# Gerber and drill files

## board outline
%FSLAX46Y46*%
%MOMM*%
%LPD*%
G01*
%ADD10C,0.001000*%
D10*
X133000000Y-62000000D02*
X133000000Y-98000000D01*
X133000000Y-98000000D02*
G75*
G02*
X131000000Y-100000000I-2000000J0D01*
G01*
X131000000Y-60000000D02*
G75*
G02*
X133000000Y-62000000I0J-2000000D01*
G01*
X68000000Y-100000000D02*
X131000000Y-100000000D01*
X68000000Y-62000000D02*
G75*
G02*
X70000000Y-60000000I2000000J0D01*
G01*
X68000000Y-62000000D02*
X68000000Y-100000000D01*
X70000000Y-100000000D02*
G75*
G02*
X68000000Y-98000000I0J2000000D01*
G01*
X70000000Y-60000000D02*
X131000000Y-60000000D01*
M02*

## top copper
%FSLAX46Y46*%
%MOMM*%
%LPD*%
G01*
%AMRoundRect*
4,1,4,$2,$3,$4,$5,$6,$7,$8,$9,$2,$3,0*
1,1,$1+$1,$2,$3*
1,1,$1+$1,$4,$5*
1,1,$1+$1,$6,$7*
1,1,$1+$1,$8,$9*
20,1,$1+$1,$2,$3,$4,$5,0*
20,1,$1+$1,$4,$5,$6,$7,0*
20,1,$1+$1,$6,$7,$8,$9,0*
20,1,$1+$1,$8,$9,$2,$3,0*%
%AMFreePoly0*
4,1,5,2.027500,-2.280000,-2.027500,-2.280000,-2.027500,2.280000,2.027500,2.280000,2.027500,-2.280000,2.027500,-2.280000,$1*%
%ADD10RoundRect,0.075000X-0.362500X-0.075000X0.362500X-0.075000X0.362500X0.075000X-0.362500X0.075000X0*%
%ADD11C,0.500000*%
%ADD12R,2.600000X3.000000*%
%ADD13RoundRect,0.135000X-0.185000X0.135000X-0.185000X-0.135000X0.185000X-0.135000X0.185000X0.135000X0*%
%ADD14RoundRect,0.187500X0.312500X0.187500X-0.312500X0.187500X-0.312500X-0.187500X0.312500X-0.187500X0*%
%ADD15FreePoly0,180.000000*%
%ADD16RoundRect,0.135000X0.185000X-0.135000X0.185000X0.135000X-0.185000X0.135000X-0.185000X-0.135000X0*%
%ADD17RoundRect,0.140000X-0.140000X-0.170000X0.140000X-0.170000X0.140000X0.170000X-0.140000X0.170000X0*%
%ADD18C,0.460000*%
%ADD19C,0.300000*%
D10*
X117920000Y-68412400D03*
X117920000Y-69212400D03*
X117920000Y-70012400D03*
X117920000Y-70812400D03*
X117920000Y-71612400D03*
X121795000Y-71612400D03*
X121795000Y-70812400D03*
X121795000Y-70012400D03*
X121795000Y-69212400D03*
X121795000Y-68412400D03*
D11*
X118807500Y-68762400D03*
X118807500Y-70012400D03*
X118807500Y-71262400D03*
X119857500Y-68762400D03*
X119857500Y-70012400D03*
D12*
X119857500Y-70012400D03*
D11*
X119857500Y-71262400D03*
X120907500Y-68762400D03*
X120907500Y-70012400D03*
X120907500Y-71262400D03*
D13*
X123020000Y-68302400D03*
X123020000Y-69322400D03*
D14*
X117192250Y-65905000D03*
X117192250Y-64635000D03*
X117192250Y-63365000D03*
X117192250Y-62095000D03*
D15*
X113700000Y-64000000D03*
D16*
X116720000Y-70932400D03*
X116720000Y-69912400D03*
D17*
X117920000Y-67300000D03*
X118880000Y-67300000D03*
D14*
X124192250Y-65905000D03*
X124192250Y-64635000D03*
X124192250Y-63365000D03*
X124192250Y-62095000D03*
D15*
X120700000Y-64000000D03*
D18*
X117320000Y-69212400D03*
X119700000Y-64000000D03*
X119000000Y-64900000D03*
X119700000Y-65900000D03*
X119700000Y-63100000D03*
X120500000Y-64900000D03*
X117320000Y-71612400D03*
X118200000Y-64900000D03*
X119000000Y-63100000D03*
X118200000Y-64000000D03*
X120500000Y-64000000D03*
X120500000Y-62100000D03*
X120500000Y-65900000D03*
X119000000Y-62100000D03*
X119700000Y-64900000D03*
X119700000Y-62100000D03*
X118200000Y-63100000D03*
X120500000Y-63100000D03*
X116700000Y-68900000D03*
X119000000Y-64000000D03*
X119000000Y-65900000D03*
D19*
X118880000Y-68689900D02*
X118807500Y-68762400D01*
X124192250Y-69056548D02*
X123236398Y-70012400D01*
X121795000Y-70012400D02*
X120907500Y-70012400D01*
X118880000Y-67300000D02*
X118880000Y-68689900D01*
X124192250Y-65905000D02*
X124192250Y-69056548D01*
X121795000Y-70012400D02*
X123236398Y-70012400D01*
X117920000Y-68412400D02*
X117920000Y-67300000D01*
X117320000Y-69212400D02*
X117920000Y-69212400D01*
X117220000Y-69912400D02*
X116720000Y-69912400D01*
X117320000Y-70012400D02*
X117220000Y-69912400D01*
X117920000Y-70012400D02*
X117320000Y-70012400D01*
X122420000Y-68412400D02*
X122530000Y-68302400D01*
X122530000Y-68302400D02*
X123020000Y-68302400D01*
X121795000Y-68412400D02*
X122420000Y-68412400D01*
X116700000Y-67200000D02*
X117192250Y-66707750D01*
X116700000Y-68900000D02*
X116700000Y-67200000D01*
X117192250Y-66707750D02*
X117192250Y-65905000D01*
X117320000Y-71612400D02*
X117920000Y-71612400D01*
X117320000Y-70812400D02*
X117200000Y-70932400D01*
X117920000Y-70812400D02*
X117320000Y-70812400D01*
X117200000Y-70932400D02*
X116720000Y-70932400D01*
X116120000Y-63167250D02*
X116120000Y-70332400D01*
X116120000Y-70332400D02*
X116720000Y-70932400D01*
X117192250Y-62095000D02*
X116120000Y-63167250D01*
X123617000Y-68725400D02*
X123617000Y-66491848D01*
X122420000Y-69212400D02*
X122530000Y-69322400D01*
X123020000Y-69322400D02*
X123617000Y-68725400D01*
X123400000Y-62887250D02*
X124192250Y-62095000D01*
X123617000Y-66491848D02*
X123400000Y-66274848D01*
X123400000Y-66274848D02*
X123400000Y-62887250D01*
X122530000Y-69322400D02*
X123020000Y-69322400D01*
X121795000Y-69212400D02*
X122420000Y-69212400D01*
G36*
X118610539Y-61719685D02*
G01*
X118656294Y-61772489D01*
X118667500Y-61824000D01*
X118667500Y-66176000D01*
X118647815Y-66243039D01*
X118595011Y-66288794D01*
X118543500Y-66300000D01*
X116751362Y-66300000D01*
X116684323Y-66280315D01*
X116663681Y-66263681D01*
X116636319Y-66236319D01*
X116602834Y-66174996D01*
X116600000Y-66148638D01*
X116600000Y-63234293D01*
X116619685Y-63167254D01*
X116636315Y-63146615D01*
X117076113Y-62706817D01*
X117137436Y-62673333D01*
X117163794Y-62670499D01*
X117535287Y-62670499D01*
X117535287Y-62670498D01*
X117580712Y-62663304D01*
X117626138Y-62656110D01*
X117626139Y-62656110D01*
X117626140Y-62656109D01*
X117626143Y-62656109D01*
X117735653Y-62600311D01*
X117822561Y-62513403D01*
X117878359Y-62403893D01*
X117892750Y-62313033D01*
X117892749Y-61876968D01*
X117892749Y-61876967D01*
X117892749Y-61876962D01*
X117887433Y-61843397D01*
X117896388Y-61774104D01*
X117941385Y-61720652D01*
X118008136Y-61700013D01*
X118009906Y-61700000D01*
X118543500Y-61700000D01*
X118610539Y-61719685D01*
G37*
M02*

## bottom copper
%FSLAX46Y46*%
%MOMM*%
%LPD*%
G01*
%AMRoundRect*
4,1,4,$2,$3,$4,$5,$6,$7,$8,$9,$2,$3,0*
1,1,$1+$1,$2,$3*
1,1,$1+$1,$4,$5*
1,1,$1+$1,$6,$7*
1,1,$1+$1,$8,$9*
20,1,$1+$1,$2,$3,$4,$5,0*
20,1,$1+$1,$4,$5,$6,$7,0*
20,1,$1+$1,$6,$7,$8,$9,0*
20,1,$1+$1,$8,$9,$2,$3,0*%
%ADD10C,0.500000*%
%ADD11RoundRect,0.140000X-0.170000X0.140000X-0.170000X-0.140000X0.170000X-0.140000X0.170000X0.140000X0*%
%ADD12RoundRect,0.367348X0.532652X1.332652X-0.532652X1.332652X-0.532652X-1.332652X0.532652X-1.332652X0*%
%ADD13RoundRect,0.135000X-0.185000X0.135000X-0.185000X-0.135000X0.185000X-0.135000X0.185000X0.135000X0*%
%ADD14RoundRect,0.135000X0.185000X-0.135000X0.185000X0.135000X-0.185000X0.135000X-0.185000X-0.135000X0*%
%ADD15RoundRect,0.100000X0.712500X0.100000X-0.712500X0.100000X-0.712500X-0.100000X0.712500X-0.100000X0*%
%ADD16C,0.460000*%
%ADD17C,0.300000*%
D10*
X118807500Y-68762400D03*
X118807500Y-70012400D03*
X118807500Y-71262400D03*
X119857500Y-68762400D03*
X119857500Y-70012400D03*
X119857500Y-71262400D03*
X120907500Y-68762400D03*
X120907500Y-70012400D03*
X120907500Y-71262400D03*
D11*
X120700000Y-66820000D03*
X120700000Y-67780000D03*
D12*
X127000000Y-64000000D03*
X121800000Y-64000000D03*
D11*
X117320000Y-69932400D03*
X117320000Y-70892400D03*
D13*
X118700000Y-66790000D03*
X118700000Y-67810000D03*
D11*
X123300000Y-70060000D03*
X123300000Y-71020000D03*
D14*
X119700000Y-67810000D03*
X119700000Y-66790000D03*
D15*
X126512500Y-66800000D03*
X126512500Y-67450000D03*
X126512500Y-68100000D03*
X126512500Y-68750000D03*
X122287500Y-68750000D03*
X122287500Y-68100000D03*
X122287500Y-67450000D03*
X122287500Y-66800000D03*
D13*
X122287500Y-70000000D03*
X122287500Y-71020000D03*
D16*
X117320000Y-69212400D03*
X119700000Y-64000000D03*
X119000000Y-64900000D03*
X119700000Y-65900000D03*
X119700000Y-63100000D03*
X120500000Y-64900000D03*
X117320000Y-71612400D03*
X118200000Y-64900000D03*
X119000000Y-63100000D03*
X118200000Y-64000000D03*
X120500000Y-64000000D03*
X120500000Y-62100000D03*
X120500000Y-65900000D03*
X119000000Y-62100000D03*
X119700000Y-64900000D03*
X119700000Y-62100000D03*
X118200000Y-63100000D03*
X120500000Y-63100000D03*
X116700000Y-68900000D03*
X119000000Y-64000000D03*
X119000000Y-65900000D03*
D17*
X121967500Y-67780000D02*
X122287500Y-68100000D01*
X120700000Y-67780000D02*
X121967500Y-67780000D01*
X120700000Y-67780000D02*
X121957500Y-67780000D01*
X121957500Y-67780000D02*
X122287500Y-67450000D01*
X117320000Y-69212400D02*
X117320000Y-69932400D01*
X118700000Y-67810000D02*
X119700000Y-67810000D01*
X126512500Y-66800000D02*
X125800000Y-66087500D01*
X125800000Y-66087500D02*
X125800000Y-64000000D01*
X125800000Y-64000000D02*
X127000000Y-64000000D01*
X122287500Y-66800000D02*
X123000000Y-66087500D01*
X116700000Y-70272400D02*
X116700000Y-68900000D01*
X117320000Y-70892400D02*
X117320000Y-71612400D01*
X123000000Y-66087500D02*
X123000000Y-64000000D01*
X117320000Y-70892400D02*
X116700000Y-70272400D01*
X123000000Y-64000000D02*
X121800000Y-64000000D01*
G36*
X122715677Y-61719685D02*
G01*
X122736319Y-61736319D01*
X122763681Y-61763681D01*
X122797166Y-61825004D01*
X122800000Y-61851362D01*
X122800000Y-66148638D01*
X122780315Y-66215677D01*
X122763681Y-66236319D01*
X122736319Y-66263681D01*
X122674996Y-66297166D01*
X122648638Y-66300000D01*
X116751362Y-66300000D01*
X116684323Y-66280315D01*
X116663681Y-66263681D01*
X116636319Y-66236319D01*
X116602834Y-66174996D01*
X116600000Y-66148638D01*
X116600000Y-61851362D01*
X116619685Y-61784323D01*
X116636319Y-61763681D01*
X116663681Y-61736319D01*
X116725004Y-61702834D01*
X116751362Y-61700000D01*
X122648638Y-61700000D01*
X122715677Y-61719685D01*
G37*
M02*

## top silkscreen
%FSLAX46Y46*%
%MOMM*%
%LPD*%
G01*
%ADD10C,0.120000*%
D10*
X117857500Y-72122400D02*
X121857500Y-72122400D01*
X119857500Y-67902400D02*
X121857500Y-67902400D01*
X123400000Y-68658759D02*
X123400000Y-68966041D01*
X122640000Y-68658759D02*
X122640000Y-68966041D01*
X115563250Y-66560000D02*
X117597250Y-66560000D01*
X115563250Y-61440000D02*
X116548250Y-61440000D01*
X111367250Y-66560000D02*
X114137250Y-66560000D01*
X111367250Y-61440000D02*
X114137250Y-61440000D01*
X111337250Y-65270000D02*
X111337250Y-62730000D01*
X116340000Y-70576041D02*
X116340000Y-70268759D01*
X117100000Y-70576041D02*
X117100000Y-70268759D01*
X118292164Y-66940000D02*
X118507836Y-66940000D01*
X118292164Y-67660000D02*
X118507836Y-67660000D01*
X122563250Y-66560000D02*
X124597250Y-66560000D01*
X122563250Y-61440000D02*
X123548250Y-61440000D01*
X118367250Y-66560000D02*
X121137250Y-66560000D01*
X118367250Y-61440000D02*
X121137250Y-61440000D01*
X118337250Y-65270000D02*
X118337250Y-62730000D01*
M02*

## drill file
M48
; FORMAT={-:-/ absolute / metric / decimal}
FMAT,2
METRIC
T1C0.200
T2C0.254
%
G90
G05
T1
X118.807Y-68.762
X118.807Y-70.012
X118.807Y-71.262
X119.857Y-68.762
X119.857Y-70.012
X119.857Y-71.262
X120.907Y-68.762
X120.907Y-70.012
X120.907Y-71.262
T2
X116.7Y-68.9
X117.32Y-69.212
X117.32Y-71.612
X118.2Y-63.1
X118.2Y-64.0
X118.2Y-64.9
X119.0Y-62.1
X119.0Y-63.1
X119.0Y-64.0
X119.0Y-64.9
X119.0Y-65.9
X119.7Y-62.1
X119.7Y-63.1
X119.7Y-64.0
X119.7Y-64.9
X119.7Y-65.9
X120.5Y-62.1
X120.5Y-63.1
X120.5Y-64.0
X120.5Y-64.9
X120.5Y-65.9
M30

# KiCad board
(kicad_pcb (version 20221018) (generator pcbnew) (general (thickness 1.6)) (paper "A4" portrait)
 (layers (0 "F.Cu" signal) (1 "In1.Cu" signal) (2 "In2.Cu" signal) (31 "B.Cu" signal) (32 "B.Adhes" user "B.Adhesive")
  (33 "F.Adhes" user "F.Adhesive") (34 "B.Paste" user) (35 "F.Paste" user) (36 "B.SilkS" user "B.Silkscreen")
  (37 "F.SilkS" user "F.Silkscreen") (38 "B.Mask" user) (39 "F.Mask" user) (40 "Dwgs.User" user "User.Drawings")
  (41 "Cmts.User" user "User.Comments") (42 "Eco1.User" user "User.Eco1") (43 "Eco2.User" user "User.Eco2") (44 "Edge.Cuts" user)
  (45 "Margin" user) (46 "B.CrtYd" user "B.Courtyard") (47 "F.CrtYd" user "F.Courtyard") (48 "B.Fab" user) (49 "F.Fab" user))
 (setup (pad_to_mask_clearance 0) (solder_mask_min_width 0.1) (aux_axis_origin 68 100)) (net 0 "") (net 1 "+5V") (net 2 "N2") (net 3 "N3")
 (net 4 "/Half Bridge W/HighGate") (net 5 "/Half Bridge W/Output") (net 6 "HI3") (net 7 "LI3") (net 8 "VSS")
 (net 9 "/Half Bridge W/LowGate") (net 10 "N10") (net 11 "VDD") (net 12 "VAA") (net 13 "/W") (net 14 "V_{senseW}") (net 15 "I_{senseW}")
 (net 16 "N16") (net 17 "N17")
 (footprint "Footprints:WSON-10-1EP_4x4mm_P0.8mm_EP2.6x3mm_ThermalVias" (layer "F.Cu") (at 119.8575 70.0124)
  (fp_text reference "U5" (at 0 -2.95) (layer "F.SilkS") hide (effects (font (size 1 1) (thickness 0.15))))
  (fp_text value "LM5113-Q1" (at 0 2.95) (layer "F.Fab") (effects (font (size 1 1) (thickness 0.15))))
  (fp_line (start -2 2.11) (end 2 2.11) (stroke (width 0.12) (type solid)) (layer "F.SilkS"))
  (fp_line (start 0 -2.11) (end 2 -2.11) (stroke (width 0.12) (type solid)) (layer "F.SilkS"))
  (pad "" smd roundrect (at -0.65 -0.75) (size 1.05 1.21) (layers "F.Paste") (roundrect_rratio 0.238095))
  (pad "" smd roundrect (at -0.65 0.75) (size 1.05 1.21) (layers "F.Paste") (roundrect_rratio 0.238095))
  (pad "" smd roundrect (at 0.65 -0.75) (size 1.05 1.21) (layers "F.Paste") (roundrect_rratio 0.238095))
  (pad "" smd roundrect (at 0.65 0.75) (size 1.05 1.21) (layers "F.Paste") (roundrect_rratio 0.238095))
  (pad "1" smd roundrect (at -1.9375 -1.6) (size 0.875 0.3) (layers "F.Cu" "F.Paste" "F.Mask") (roundrect_rratio 0.25) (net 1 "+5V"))
  (pad "2" smd roundrect (at -1.9375 -0.8) (size 0.875 0.3) (layers "F.Cu" "F.Paste" "F.Mask") (roundrect_rratio 0.25) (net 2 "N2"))
  (pad "3" smd roundrect (at -1.9375 0) (size 0.875 0.3) (layers "F.Cu" "F.Paste" "F.Mask") (roundrect_rratio 0.25) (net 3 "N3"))
  (pad "4" smd roundrect (at -1.9375 0.8) (size 0.875 0.3) (layers "F.Cu" "F.Paste" "F.Mask") (roundrect_rratio 0.25)
   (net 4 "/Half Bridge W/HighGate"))
  (pad "5" smd roundrect (at -1.9375 1.6) (size 0.875 0.3) (layers "F.Cu" "F.Paste" "F.Mask") (roundrect_rratio 0.25)
   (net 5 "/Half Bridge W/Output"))
  (pad "6" smd roundrect (at 1.9375 1.6) (size 0.875 0.3) (layers "F.Cu" "F.Paste" "F.Mask") (roundrect_rratio 0.25) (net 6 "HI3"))
  (pad "7" smd roundrect (at 1.9375 0.8) (size 0.875 0.3) (layers "F.Cu" "F.Paste" "F.Mask") (roundrect_rratio 0.25) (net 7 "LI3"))
  (pad "8" smd roundrect (at 1.9375 0) (size 0.875 0.3) (layers "F.Cu" "F.Paste" "F.Mask") (roundrect_rratio 0.25) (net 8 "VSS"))
  (pad "9" smd roundrect (at 1.9375 -0.8) (size 0.875 0.3) (layers "F.Cu" "F.Paste" "F.Mask") (roundrect_rratio 0.25)
   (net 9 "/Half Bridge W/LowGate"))
  (pad "10" smd roundrect (at 1.9375 -1.6) (size 0.875 0.3) (layers "F.Cu" "F.Paste" "F.Mask") (roundrect_rratio 0.25) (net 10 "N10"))
  (pad "11" thru_hole circle (at -1.05 -1.25) (size 0.5 0.5) (drill 0.2) (layers "*.Cu") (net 8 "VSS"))
  (pad "11" thru_hole circle (at -1.05 0) (size 0.5 0.5) (drill 0.2) (layers "*.Cu") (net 8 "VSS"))
  (pad "11" thru_hole circle (at -1.05 1.25) (size 0.5 0.5) (drill 0.2) (layers "*.Cu") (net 8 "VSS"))
  (pad "11" thru_hole circle (at 0 -1.25) (size 0.5 0.5) (drill 0.2) (layers "*.Cu") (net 8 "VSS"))
  (pad "11" thru_hole circle (at 0 0) (size 0.5 0.5) (drill 0.2) (layers "*.Cu") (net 8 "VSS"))
  (pad "11" smd rect (at 0 0) (size 2.6 3) (layers "F.Cu" "F.Mask") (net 8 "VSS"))
  (pad "11" thru_hole circle (at 0 1.25) (size 0.5 0.5) (drill 0.2) (layers "*.Cu") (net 8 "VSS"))
  (pad "11" thru_hole circle (at 1.05 -1.25) (size 0.5 0.5) (drill 0.2) (layers "*.Cu") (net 8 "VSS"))
  (pad "11" thru_hole circle (at 1.05 0) (size 0.5 0.5) (drill 0.2) (layers "*.Cu") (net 8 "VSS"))
  (pad "11" thru_hole circle (at 1.05 1.25) (size 0.5 0.5) (drill 0.2) (layers "*.Cu") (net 8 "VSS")))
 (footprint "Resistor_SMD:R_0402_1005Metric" (layer "F.Cu") (at 123.02 68.8124 -90)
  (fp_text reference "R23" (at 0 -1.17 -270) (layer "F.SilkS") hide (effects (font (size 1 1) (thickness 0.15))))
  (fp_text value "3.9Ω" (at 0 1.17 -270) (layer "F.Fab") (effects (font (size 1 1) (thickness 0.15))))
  (fp_line (start -0.153641 -0.38) (end 0.153641 -0.38) (stroke (width 0.12) (type solid)) (layer "F.SilkS"))
  (fp_line (start -0.153641 0.38) (end 0.153641 0.38) (stroke (width 0.12) (type solid)) (layer "F.SilkS"))
  (pad "1" smd roundrect (at -0.51 0 270) (size 0.54 0.64) (layers "F.Cu" "F.Paste" "F.Mask") (roundrect_rratio 0.25) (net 10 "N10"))
  (pad "2" smd roundrect (at 0.51 0 270) (size 0.54 0.64) (layers "F.Cu" "F.Paste" "F.Mask") (roundrect_rratio 0.25)
   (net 9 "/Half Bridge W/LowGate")))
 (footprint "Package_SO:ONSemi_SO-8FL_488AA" (layer "F.Cu") (at 114.445 64 180)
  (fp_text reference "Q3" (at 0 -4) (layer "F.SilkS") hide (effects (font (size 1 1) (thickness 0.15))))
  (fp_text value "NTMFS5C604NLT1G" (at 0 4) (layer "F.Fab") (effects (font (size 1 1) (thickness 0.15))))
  (fp_line (start -1.11825 -2.56) (end -3.15225 -2.56) (stroke (width 0.12) (type solid)) (layer "F.SilkS"))
  (fp_line (start -1.11825 2.56) (end -2.10325 2.56) (stroke (width 0.12) (type solid)) (layer "F.SilkS"))
  (fp_line (start 3.07775 -2.56) (end 0.30775 -2.56) (stroke (width 0.12) (type solid)) (layer "F.SilkS"))
  (fp_line (start 3.07775 2.56) (end 0.30775 2.56) (stroke (width 0.12) (type solid)) (layer "F.SilkS"))
  (fp_line (start 3.10775 -1.27) (end 3.10775 1.27) (stroke (width 0.12) (type solid)) (layer "F.SilkS"))
  (pad "1" smd roundrect (at -2.74725 -1.905 180) (size 1 0.75) (layers "F.Cu" "F.Paste" "F.Mask") (roundrect_rratio 0.25)
   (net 5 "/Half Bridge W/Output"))
  (pad "2" smd roundrect (at -2.74725 -0.635 180) (size 1 0.75) (layers "F.Cu" "F.Paste" "F.Mask") (roundrect_rratio 0.25)
   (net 5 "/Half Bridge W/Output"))
  (pad "3" smd roundrect (at -2.74725 0.635 180) (size 1 0.75) (layers "F.Cu" "F.Paste" "F.Mask") (roundrect_rratio 0.25)
   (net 5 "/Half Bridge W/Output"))
  (pad "4" smd roundrect (at -2.74725 1.905 180) (size 1 0.75) (layers "F.Cu" "F.Paste" "F.Mask") (roundrect_rratio 0.25)
   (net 4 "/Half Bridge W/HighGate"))
  (pad "5" smd custom (at 0.745 0 180) (size 4.055 4.56) (layers "F.Cu" "F.Paste" "F.Mask") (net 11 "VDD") (zone_connect 0)
   (options (clearance outline) (anchor rect)) (primitives)))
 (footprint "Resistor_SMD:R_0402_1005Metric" (layer "F.Cu") (at 116.72 70.4224 90)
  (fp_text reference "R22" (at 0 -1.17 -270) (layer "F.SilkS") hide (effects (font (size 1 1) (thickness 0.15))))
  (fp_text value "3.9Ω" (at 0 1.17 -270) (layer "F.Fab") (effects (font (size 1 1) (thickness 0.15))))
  (fp_line (start -0.153641 -0.38) (end 0.153641 -0.38) (stroke (width 0.12) (type solid)) (layer "F.SilkS"))
  (fp_line (start -0.153641 0.38) (end 0.153641 0.38) (stroke (width 0.12) (type solid)) (layer "F.SilkS"))
  (pad "1" smd roundrect (at -0.51 0 90) (size 0.54 0.64) (layers "F.Cu" "F.Paste" "F.Mask") (roundrect_rratio 0.25)
   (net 4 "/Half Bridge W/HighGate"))
  (pad "2" smd roundrect (at 0.51 0 90) (size 0.54 0.64) (layers "F.Cu" "F.Paste" "F.Mask") (roundrect_rratio 0.25) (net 3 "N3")))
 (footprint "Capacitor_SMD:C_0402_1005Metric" (layer "F.Cu") (at 118.4 67.3)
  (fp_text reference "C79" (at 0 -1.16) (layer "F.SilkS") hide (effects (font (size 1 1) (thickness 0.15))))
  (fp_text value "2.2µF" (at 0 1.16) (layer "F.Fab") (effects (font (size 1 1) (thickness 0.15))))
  (fp_line (start -0.107836 -0.36) (end 0.107836 -0.36) (stroke (width 0.12) (type solid)) (layer "F.SilkS"))
  (fp_line (start -0.107836 0.36) (end 0.107836 0.36) (stroke (width 0.12) (type solid)) (layer "F.SilkS"))
  (pad "1" smd roundrect (at -0.48 0) (size 0.56 0.62) (layers "F.Cu" "F.Paste" "F.Mask") (roundrect_rratio 0.25) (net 1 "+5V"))
  (pad "2" smd roundrect (at 0.48 0) (size 0.56 0.62) (layers "F.Cu" "F.Paste" "F.Mask") (roundrect_rratio 0.25) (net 8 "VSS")))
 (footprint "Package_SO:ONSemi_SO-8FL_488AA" (layer "F.Cu") (at 121.445 64 180)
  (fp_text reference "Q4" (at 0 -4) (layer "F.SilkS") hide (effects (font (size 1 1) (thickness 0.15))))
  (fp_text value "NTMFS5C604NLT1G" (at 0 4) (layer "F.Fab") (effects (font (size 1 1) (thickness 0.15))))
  (fp_line (start -1.11825 -2.56) (end -3.15225 -2.56) (stroke (width 0.12) (type solid)) (layer "F.SilkS"))
  (fp_line (start -1.11825 2.56) (end -2.10325 2.56) (stroke (width 0.12) (type solid)) (layer "F.SilkS"))
  (fp_line (start 3.07775 -2.56) (end 0.30775 -2.56) (stroke (width 0.12) (type solid)) (layer "F.SilkS"))
  (fp_line (start 3.07775 2.56) (end 0.30775 2.56) (stroke (width 0.12) (type solid)) (layer "F.SilkS"))
  (fp_line (start 3.10775 -1.27) (end 3.10775 1.27) (stroke (width 0.12) (type solid)) (layer "F.SilkS"))
  (pad "1" smd roundrect (at -2.74725 -1.905 180) (size 1 0.75) (layers "F.Cu" "F.Paste" "F.Mask") (roundrect_rratio 0.25) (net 8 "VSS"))
  (pad "2" smd roundrect (at -2.74725 -0.635 180) (size 1 0.75) (layers "F.Cu" "F.Paste" "F.Mask") (roundrect_rratio 0.25) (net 8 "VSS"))
  (pad "3" smd roundrect (at -2.74725 0.635 180) (size 1 0.75) (layers "F.Cu" "F.Paste" "F.Mask") (roundrect_rratio 0.25) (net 8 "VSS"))
  (pad "4" smd roundrect (at -2.74725 1.905 180) (size 1 0.75) (layers "F.Cu" "F.Paste" "F.Mask") (roundrect_rratio 0.25)
   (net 9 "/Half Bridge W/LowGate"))
  (pad "5" smd custom (at 0.745 0 180) (size 4.055 4.56) (layers "F.Cu" "F.Paste" "F.Mask") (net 5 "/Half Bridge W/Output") (zone_connect 0)
   (options (clearance outline) (anchor rect)) (primitives)))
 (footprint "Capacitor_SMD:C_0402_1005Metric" (layer "B.Cu") (at 120.7 67.3 -90)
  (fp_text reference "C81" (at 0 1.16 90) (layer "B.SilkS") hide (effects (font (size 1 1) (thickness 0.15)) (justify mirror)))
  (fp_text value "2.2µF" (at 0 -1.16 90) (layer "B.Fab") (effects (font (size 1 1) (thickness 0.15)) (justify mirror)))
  (pad "1" smd roundrect (at -0.48 0 270) (size 0.56 0.62) (layers "B.Cu" "B.Paste" "B.Mask") (roundrect_rratio 0.25) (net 8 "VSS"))
  (pad "2" smd roundrect (at 0.48 0 270) (size 0.56 0.62) (layers "B.Cu" "B.Paste" "B.Mask") (roundrect_rratio 0.25) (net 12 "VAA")))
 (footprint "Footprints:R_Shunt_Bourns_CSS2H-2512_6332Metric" (layer "B.Cu") (at 124.4 64 180)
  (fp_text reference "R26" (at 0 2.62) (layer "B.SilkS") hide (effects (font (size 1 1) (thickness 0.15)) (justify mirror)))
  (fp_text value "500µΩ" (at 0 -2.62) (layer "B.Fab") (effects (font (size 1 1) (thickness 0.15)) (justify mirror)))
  (pad "1" smd roundrect (at -2.6 0 180) (size 1.8 3.4) (layers "B.Cu" "B.Paste" "B.Mask") (roundrect_rratio 0.204082) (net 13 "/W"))
  (pad "2" smd roundrect (at 2.6 0 180) (size 1.8 3.4) (layers "B.Cu" "B.Paste" "B.Mask") (roundrect_rratio 0.204082)
   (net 5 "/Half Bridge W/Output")))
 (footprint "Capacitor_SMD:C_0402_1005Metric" (layer "B.Cu") (at 117.32 70.4124 -90)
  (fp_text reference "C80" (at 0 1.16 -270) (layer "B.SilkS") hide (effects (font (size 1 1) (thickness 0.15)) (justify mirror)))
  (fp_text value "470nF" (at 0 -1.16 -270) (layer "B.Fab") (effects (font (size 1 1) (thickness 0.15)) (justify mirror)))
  (pad "1" smd roundrect (at -0.48 0 270) (size 0.56 0.62) (layers "B.Cu" "B.Paste" "B.Mask") (roundrect_rratio 0.25) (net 2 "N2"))
  (pad "2" smd roundrect (at 0.48 0 270) (size 0.56 0.62) (layers "B.Cu" "B.Paste" "B.Mask") (roundrect_rratio 0.25)
   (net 5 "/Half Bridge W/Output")))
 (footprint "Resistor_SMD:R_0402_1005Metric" (layer "B.Cu") (at 118.7 67.3 -90)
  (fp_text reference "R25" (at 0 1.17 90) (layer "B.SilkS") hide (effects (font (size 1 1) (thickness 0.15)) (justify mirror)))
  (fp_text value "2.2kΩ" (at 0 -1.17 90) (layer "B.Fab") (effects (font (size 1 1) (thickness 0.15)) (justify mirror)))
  (pad "1" smd roundrect (at -0.51 0 270) (size 0.54 0.64) (layers "B.Cu" "B.Paste" "B.Mask") (roundrect_rratio 0.25) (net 8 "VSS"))
  (pad "2" smd roundrect (at 0.51 0 270) (size 0.54 0.64) (layers "B.Cu" "B.Paste" "B.Mask") (roundrect_rratio 0.25) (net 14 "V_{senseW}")))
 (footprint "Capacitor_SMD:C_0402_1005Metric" (layer "B.Cu") (at 123.3 70.54 -90)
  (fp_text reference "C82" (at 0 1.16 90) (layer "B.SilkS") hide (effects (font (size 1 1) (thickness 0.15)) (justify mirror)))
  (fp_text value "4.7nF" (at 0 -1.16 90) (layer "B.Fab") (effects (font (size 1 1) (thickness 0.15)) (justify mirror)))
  (pad "1" smd roundrect (at -0.48 0 270) (size 0.56 0.62) (layers "B.Cu" "B.Paste" "B.Mask") (roundrect_rratio 0.25) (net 8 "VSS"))
  (pad "2" smd roundrect (at 0.48 0 270) (size 0.56 0.62) (layers "B.Cu" "B.Paste" "B.Mask") (roundrect_rratio 0.25) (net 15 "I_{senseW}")))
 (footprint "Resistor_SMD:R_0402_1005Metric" (layer "B.Cu") (at 119.7 67.3 90)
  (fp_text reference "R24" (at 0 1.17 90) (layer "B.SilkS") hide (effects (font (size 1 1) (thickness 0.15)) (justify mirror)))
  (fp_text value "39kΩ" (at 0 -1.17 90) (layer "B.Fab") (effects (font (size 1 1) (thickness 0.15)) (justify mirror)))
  (pad "1" smd roundrect (at -0.51 0 90) (size 0.54 0.64) (layers "B.Cu" "B.Paste" "B.Mask") (roundrect_rratio 0.25) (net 14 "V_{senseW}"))
  (pad "2" smd roundrect (at 0.51 0 90) (size 0.54 0.64) (layers "B.Cu" "B.Paste" "B.Mask") (roundrect_rratio 0.25)
   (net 5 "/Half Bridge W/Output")))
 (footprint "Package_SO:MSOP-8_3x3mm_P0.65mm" (layer "B.Cu") (at 124.4 67.775 180)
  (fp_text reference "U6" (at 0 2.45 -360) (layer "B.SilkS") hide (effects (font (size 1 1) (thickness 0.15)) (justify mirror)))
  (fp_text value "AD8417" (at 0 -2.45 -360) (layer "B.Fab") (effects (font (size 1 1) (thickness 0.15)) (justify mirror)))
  (pad "1" smd roundrect (at -2.1125 0.975 180) (size 1.625 0.4) (layers "B.Cu" "B.Paste" "B.Mask") (roundrect_rratio 0.25) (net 13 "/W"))
  (pad "2" smd roundrect (at -2.1125 0.325 180) (size 1.625 0.4) (layers "B.Cu" "B.Paste" "B.Mask") (roundrect_rratio 0.25) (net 8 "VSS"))
  (pad "3" smd roundrect (at -2.1125 -0.325 180) (size 1.625 0.4) (layers "B.Cu" "B.Paste" "B.Mask") (roundrect_rratio 0.25) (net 8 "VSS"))
  (pad "4" smd roundrect (at -2.1125 -0.975 180) (size 1.625 0.4) (layers "B.Cu" "B.Paste" "B.Mask") (roundrect_rratio 0.25) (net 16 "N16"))
  (pad "5" smd roundrect (at 2.1125 -0.975 180) (size 1.625 0.4) (layers "B.Cu" "B.Paste" "B.Mask") (roundrect_rratio 0.25) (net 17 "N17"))
  (pad "6" smd roundrect (at 2.1125 -0.325 180) (size 1.625 0.4) (layers "B.Cu" "B.Paste" "B.Mask") (roundrect_rratio 0.25) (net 12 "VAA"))
  (pad "7" smd roundrect (at 2.1125 0.325 180) (size 1.625 0.4) (layers "B.Cu" "B.Paste" "B.Mask") (roundrect_rratio 0.25) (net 12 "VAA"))
  (pad "8" smd roundrect (at 2.1125 0.975 180) (size 1.625 0.4) (layers "B.Cu" "B.Paste" "B.Mask") (roundrect_rratio 0.25)
   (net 5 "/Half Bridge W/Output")))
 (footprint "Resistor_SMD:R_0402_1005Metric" (layer "B.Cu") (at 122.2875 70.51 -90)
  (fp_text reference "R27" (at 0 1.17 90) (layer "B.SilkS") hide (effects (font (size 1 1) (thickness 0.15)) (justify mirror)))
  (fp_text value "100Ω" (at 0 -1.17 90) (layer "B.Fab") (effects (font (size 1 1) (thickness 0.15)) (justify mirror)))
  (pad "1" smd roundrect (at -0.51 0 270) (size 0.54 0.64) (layers "B.Cu" "B.Paste" "B.Mask") (roundrect_rratio 0.25) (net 17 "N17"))
  (pad "2" smd roundrect (at 0.51 0 270) (size 0.54 0.64) (layers "B.Cu" "B.Paste" "B.Mask") (roundrect_rratio 0.25) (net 15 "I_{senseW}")))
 (gr_line (start 133 62) (end 133 98) (stroke (width 0.001) (type solid)) (layer "Edge.Cuts"))
 (gr_arc (start 133 98) (mid 132.414214 99.414214) (end 131 100) (stroke (width 0.001) (type solid)) (layer "Edge.Cuts"))
 (gr_arc (start 131 60) (mid 132.414214 60.585786) (end 133 62) (stroke (width 0.001) (type solid)) (layer "Edge.Cuts"))
 (gr_line (start 68 100) (end 131 100) (stroke (width 0.001) (type solid)) (layer "Edge.Cuts"))
 (gr_arc (start 68 62) (mid 68.585786 60.585786) (end 70 60) (stroke (width 0.001) (type solid)) (layer "Edge.Cuts"))
 (gr_line (start 68 62) (end 68 100) (stroke (width 0.001) (type solid)) (layer "Edge.Cuts"))
 (gr_arc (start 70 100) (mid 68.585786 99.414214) (end 68 98) (stroke (width 0.001) (type solid)) (layer "Edge.Cuts"))
 (gr_line (start 70 60) (end 131 60) (stroke (width 0.001) (type solid)) (layer "Edge.Cuts"))
 (segment (start 118.88 68.6899) (end 118.8075 68.7624) (width 0.3) (layer "F.Cu") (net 8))
 (segment (start 124.19225 69.056548) (end 123.236398 70.0124) (width 0.3) (layer "F.Cu") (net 8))
 (segment (start 121.795 70.0124) (end 120.9075 70.0124) (width 0.3) (layer "F.Cu") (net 8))
 (segment (start 118.88 67.3) (end 118.88 68.6899) (width 0.3) (layer "F.Cu") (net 8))
 (segment (start 124.19225 65.905) (end 124.19225 69.056548) (width 0.3) (layer "F.Cu") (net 8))
 (segment (start 121.795 70.0124) (end 123.236398 70.0124) (width 0.3) (layer "F.Cu") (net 8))
 (segment (start 117.92 68.4124) (end 117.92 67.3) (width 0.3) (layer "F.Cu") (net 1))
 (segment (start 121.9675 67.78) (end 122.2875 68.1) (width 0.3) (layer "B.Cu") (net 12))
 (segment (start 120.7 67.78) (end 121.9675 67.78) (width 0.3) (layer "B.Cu") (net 12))
 (segment (start 120.7 67.78) (end 121.9575 67.78) (width 0.3) (layer "B.Cu") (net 12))
 (segment (start 121.9575 67.78) (end 122.2875 67.45) (width 0.3) (layer "B.Cu") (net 12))
 (segment (start 117.32 69.2124) (end 117.92 69.2124) (width 0.3) (layer "F.Cu") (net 2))
 (via (at 117.32 69.2124) (size 0.46) (drill 0.254) (layers "F.Cu" "B.Cu") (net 2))
 (segment (start 117.32 69.2124) (end 117.32 69.9324) (width 0.3) (layer "B.Cu") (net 2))
 (segment (start 117.22 69.9124) (end 116.72 69.9124) (width 0.3) (layer "F.Cu") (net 3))
 (segment (start 117.32 70.0124) (end 117.22 69.9124) (width 0.3) (layer "F.Cu") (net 3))
 (segment (start 117.92 70.0124) (end 117.32 70.0124) (width 0.3) (layer "F.Cu") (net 3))
 (segment (start 122.42 68.4124) (end 122.53 68.3024) (width 0.3) (layer "F.Cu") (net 10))
 (segment (start 122.53 68.3024) (end 123.02 68.3024) (width 0.3) (layer "F.Cu") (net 10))
 (segment (start 121.795 68.4124) (end 122.42 68.4124) (width 0.3) (layer "F.Cu") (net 10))
 (segment (start 118.7 67.81) (end 119.7 67.81) (width 0.3) (layer "B.Cu") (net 14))
 (segment (start 126.5125 66.8) (end 125.8 66.0875) (width 0.3) (layer "B.Cu") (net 13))
 (segment (start 125.8 66.0875) (end 125.8 64) (width 0.3) (layer "B.Cu") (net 13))
 (segment (start 125.8 64) (end 127 64) (width 0.3) (layer "B.Cu") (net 13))
 (segment (start 116.7 67.2) (end 117.19225 66.70775) (width 0.3) (layer "F.Cu") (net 5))
 (segment (start 116.7 68.9) (end 116.7 67.2) (width 0.3) (layer "F.Cu") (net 5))
 (segment (start 117.19225 66.70775) (end 117.19225 65.905) (width 0.3) (layer "F.Cu") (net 5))
 (segment (start 117.32 71.6124) (end 117.92 71.6124) (width 0.3) (layer "F.Cu") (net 5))
 (via (at 119.7 64) (size 0.46) (drill 0.254) (layers "F.Cu" "B.Cu") (free) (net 5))
 (via (at 119 64.9) (size 0.46) (drill 0.254) (layers "F.Cu" "B.Cu") (free) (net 5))
 (via (at 119.7 65.9) (size 0.46) (drill 0.254) (layers "F.Cu" "B.Cu") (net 5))
 (via (at 119.7 63.1) (size 0.46) (drill 0.254) (layers "F.Cu" "B.Cu") (free) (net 5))
 (via (at 120.5 64.9) (size 0.46) (drill 0.254) (layers "F.Cu" "B.Cu") (free) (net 5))
 (via (at 117.32 71.6124) (size 0.46) (drill 0.254) (layers "F.Cu" "B.Cu") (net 5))
 (via (at 118.2 64.9) (size 0.46) (drill 0.254) (layers "F.Cu" "B.Cu") (free) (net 5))
 (via (at 119 63.1) (size 0.46) (drill 0.254) (layers "F.Cu" "B.Cu") (free) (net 5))
 (via (at 118.2 64) (size 0.46) (drill 0.254) (layers "F.Cu" "B.Cu") (free) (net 5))
 (via (at 120.5 64) (size 0.46) (drill 0.254) (layers "F.Cu" "B.Cu") (free) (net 5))
 (via (at 120.5 62.1) (size 0.46) (drill 0.254) (layers "F.Cu" "B.Cu") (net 5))
 (via (at 120.5 65.9) (size 0.46) (drill 0.254) (layers "F.Cu" "B.Cu") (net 5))
 (via (at 119 62.1) (size 0.46) (drill 0.254) (layers "F.Cu" "B.Cu") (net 5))
 (via (at 119.7 64.9) (size 0.46) (drill 0.254) (layers "F.Cu" "B.Cu") (free) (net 5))
 (via (at 119.7 62.1) (size 0.46) (drill 0.254) (layers "F.Cu" "B.Cu") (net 5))
 (via (at 118.2 63.1) (size 0.46) (drill 0.254) (layers "F.Cu" "B.Cu") (free) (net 5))
 (via (at 120.5 63.1) (size 0.46) (drill 0.254) (layers "F.Cu" "B.Cu") (free) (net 5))
 (via (at 116.7 68.9) (size 0.46) (drill 0.254) (layers "F.Cu" "B.Cu") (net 5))
 (via (at 119 64) (size 0.46) (drill 0.254) (layers "F.Cu" "B.Cu") (free) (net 5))
 (via (at 119 65.9) (size 0.46) (drill 0.254) (layers "F.Cu" "B.Cu") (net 5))
 (segment (start 122.2875 66.8) (end 123 66.0875) (width 0.3) (layer "B.Cu") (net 5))
 (segment (start 116.7 70.2724) (end 116.7 68.9) (width 0.3) (layer "B.Cu") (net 5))
 (segment (start 117.32 70.8924) (end 117.32 71.6124) (width 0.3) (layer "B.Cu") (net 5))
 (segment (start 123 66.0875) (end 123 64) (width 0.3) (layer "B.Cu") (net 5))
 (segment (start 117.32 70.8924) (end 116.7 70.2724) (width 0.3) (layer "B.Cu") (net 5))
 (segment (start 123 64) (end 121.8 64) (width 0.3) (layer "B.Cu") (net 5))
 (segment (start 117.32 70.8124) (end 117.2 70.9324) (width 0.3) (layer "F.Cu") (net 4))
 (segment (start 117.92 70.8124) (end 117.32 70.8124) (width 0.3) (layer "F.Cu") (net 4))
 (segment (start 117.2 70.9324) (end 116.72 70.9324) (width 0.3) (layer "F.Cu") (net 4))
 (segment (start 116.12 63.16725) (end 116.12 70.3324) (width 0.3) (layer "F.Cu") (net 4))
 (segment (start 116.12 70.3324) (end 116.72 70.9324) (width 0.3) (layer "F.Cu") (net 4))
 (segment (start 117.19225 62.095) (end 116.12 63.16725) (width 0.3) (layer "F.Cu") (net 4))
 (segment (start 123.617 68.7254) (end 123.617 66.491848) (width 0.3) (layer "F.Cu") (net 9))
 (segment (start 122.42 69.2124) (end 122.53 69.3224) (width 0.3) (layer "F.Cu") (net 9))
 (segment (start 123.02 69.3224) (end 123.617 68.7254) (width 0.3) (layer "F.Cu") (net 9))
 (segment (start 123.4 62.88725) (end 124.19225 62.095) (width 0.3) (layer "F.Cu") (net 9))
 (segment (start 123.617 66.491848) (end 123.4 66.274848) (width 0.3) (layer "F.Cu") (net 9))
 (segment (start 123.4 66.274848) (end 123.4 62.88725) (width 0.3) (layer "F.Cu") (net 9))
 (segment (start 122.53 69.3224) (end 123.02 69.3224) (width 0.3) (layer "F.Cu") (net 9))
 (segment (start 121.795 69.2124) (end 122.42 69.2124) (width 0.3) (layer "F.Cu") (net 9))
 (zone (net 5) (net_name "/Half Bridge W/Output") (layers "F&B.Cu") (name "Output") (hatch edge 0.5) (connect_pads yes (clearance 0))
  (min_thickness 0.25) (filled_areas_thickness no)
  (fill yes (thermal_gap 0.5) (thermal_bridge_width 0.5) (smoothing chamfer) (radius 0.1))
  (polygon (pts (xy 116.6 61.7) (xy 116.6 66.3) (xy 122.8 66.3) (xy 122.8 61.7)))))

